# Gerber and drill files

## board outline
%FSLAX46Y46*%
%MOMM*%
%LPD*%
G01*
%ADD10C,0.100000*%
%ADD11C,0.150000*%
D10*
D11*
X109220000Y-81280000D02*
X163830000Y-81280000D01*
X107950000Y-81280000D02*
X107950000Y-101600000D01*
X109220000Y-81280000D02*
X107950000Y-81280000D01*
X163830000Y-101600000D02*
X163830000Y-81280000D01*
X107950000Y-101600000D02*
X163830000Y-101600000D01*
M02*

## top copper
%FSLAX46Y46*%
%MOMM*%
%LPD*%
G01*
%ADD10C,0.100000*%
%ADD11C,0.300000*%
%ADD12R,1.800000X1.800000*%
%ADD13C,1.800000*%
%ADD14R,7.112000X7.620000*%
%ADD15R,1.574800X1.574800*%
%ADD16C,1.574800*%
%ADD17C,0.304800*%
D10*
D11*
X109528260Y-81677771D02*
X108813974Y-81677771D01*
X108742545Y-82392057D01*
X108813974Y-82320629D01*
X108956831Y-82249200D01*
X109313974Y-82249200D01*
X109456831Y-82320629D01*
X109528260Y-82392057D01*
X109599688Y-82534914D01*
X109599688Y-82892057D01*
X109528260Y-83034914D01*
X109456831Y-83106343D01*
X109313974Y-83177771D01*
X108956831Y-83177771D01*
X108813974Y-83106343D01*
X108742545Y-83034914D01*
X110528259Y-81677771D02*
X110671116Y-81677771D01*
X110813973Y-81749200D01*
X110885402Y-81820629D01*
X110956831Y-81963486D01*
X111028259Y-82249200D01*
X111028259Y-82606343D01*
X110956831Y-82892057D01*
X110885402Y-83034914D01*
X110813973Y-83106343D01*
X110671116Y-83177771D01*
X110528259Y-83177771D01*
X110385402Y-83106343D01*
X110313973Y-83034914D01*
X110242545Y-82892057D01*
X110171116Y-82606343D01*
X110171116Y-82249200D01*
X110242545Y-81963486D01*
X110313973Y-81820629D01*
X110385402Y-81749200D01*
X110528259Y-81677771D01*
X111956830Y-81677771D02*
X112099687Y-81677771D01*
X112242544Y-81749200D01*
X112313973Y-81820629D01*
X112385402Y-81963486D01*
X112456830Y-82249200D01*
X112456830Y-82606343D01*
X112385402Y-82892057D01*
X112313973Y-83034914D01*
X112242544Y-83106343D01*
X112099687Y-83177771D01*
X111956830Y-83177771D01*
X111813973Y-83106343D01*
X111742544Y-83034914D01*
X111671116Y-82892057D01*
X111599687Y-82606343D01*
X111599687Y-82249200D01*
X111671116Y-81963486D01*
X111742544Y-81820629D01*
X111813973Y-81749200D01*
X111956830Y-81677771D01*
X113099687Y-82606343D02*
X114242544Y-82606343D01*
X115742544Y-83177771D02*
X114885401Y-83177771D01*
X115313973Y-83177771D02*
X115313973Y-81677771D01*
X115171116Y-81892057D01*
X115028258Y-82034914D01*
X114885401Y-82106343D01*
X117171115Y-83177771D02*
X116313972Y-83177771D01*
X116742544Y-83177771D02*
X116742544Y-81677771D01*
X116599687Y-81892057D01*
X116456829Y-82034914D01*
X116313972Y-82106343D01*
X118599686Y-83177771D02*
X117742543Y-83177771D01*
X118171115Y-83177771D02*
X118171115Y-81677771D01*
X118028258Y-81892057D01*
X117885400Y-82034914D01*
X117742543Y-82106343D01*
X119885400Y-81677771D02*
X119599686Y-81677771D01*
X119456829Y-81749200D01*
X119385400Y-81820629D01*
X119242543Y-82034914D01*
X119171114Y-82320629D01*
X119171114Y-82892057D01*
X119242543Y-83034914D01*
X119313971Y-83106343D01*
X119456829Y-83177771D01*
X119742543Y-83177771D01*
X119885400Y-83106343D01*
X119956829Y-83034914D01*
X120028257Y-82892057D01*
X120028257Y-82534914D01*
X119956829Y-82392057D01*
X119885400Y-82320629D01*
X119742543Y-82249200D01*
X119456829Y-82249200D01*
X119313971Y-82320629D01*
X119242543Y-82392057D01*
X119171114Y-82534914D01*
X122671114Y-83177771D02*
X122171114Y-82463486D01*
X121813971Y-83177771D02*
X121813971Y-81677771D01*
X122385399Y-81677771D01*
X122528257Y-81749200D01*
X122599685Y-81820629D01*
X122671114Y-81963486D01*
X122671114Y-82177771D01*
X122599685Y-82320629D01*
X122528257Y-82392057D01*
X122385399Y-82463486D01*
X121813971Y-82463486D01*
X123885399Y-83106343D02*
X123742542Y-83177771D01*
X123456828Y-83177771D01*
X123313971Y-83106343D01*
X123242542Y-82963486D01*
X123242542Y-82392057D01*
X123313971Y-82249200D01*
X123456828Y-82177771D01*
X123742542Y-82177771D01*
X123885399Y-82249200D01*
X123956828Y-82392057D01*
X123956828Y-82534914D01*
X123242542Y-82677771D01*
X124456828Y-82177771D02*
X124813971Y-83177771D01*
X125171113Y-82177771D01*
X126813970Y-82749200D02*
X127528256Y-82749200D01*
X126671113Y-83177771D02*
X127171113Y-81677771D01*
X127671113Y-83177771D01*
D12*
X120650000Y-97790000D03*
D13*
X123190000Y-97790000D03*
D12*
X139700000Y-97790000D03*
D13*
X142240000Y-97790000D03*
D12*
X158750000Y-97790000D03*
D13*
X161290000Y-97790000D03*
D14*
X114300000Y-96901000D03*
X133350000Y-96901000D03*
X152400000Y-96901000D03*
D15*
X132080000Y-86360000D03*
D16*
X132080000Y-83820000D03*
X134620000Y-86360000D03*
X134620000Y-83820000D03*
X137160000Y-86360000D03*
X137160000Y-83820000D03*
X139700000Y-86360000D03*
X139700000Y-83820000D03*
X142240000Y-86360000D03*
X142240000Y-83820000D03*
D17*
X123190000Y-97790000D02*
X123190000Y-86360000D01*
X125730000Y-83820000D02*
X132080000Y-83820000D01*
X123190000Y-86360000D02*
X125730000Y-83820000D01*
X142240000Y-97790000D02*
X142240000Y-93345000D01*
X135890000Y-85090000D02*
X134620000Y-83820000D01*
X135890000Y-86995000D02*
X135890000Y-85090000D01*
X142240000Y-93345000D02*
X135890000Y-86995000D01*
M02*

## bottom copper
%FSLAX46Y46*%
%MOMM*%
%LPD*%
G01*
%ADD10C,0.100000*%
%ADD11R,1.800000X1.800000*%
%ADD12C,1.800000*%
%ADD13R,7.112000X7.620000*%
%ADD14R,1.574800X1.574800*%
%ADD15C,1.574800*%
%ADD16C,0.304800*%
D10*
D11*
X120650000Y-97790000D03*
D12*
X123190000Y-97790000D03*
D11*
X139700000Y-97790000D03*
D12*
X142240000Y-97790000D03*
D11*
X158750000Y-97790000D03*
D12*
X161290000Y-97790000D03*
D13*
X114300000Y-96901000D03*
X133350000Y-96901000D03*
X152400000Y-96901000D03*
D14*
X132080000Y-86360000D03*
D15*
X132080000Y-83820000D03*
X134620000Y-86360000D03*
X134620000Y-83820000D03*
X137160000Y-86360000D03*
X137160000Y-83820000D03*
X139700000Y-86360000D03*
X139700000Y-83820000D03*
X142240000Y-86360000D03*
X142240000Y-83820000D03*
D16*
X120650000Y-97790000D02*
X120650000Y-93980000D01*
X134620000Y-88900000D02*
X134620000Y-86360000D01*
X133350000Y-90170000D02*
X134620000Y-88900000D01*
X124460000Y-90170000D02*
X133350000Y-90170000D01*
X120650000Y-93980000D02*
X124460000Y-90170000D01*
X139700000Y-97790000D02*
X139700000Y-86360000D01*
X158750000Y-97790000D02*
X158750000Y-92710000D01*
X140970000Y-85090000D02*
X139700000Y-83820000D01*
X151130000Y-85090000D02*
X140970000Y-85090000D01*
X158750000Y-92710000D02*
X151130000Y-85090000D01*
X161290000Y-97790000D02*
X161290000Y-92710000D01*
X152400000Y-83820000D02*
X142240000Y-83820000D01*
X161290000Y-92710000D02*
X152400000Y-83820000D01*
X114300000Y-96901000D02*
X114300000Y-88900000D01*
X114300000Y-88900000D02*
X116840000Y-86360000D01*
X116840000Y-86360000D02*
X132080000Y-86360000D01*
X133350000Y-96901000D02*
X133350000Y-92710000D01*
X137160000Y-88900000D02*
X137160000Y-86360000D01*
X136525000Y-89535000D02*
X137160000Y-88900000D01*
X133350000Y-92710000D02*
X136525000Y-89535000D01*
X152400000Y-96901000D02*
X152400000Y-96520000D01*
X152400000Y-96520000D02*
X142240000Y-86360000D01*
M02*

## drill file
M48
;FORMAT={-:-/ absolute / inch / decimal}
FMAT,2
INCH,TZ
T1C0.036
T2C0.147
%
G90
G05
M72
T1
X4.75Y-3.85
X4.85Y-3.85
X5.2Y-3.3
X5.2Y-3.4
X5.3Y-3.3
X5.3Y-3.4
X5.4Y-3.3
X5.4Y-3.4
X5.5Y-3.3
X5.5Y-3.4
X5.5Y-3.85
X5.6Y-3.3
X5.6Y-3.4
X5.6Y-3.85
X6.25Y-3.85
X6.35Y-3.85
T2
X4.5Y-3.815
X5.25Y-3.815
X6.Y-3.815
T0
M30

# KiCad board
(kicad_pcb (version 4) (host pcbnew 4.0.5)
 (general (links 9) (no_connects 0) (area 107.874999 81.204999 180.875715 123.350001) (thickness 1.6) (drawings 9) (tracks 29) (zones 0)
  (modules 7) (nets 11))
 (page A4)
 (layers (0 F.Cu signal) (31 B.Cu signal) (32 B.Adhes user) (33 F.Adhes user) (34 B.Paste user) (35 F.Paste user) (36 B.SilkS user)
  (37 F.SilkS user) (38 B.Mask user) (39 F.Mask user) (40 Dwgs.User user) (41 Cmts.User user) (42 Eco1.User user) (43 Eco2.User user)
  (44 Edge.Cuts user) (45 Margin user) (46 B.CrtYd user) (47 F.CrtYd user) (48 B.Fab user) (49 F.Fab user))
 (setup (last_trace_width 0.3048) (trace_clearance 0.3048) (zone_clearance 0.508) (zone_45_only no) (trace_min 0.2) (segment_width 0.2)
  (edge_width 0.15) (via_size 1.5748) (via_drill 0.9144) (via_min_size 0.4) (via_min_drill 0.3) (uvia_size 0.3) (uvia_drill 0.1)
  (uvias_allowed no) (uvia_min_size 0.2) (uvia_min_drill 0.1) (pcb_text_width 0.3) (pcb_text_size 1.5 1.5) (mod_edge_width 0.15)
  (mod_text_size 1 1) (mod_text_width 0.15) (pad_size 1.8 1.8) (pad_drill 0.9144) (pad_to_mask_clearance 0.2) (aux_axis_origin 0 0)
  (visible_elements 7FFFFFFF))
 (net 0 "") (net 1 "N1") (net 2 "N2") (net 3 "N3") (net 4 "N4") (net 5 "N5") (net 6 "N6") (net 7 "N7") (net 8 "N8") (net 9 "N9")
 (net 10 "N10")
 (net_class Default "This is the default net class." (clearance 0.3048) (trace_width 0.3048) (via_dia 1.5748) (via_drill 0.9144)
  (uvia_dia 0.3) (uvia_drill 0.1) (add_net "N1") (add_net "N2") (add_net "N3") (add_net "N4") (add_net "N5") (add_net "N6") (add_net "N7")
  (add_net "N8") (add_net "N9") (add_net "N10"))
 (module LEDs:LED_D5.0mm (layer F.Cu) (at 120.65 97.79)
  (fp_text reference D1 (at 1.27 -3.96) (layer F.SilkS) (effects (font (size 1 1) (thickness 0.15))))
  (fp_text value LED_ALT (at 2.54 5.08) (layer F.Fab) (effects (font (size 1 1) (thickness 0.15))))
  (pad 1 thru_hole rect (at 0 0) (size 1.8 1.8) (drill 0.9144) (layers *.Cu *.Mask) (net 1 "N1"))
  (pad 2 thru_hole circle (at 2.54 0) (size 1.8 1.8) (drill 0.9144) (layers *.Cu *.Mask) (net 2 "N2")))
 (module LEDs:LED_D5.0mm (layer F.Cu) (at 139.7 97.79)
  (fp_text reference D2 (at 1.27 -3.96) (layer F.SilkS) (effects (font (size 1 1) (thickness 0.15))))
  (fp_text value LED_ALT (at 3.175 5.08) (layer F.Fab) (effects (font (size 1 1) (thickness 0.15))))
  (pad 1 thru_hole rect (at 0 0) (size 1.8 1.8) (drill 0.9144) (layers *.Cu *.Mask) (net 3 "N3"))
  (pad 2 thru_hole circle (at 2.54 0) (size 1.8 1.8) (drill 0.9144) (layers *.Cu *.Mask) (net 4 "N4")))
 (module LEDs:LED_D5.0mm (layer F.Cu) (at 158.75 97.79)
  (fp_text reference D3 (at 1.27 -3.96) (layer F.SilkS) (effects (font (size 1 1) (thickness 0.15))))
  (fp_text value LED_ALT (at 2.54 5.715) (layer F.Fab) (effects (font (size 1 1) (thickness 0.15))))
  (pad 1 thru_hole rect (at 0 0) (size 1.8 1.8) (drill 0.9144) (layers *.Cu *.Mask) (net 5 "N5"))
  (pad 2 thru_hole circle (at 2.54 0) (size 1.8 1.8) (drill 0.9144) (layers *.Cu *.Mask) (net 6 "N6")))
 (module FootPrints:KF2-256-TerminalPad (layer F.Cu) (at 114.3 101.6)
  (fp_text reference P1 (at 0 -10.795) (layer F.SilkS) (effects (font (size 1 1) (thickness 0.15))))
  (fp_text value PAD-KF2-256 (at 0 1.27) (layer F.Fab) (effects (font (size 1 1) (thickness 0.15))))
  (pad 1 thru_hole rect (at 0 -4.699) (size 7.112 7.62) (drill 3.7338) (layers *.Cu *.Mask F.SilkS) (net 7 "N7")))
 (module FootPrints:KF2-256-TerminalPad (layer F.Cu) (at 133.35 101.6)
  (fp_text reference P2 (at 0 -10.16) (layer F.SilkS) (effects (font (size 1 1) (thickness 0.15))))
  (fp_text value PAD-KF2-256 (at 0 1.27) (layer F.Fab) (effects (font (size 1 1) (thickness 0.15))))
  (pad 1 thru_hole rect (at 0 -4.699) (size 7.112 7.62) (drill 3.7338) (layers *.Cu *.Mask F.SilkS) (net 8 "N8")))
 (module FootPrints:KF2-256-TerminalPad (layer F.Cu) (at 152.4 101.6)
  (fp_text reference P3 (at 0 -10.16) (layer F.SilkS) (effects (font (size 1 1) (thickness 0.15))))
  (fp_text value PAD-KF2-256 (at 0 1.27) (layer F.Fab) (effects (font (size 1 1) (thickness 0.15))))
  (pad 1 thru_hole rect (at 0 -4.699) (size 7.112 7.62) (drill 3.7338) (layers *.Cu *.Mask F.SilkS) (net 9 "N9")))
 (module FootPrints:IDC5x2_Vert (layer F.Cu) (at 137.16 85.09 180)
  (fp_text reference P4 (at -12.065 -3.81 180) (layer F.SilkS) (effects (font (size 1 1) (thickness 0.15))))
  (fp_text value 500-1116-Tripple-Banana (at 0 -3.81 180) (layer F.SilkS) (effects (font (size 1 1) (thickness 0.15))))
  (pad 1 thru_hole rect (at 5.08 -1.27 180) (size 1.5748 1.5748) (drill 0.9144) (layers *.Cu *.Mask F.SilkS) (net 7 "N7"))
  (pad 2 thru_hole circle (at 5.08 1.27 180) (size 1.5748 1.5748) (drill 0.9144) (layers *.Cu *.Mask F.SilkS) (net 2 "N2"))
  (pad 3 thru_hole circle (at 2.54 -1.27 180) (size 1.5748 1.5748) (drill 0.9144) (layers *.Cu *.Mask F.SilkS) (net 1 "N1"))
  (pad 4 thru_hole circle (at 2.54 1.27 180) (size 1.5748 1.5748) (drill 0.9144) (layers *.Cu *.Mask F.SilkS) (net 4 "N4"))
  (pad 5 thru_hole circle (at 0 -1.27 180) (size 1.5748 1.5748) (drill 0.9144) (layers *.Cu *.Mask F.SilkS) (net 8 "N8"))
  (pad 6 thru_hole circle (at 0 1.27 180) (size 1.5748 1.5748) (drill 0.9144) (layers *.Cu *.Mask F.SilkS) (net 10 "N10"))
  (pad 7 thru_hole circle (at -2.54 -1.27 180) (size 1.5748 1.5748) (drill 0.9144) (layers *.Cu *.Mask F.SilkS) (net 3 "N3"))
  (pad 8 thru_hole circle (at -2.54 1.27 180) (size 1.5748 1.5748) (drill 0.9144) (layers *.Cu *.Mask F.SilkS) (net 5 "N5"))
  (pad 9 thru_hole circle (at -5.08 -1.27 180) (size 1.5748 1.5748) (drill 0.9144) (layers *.Cu *.Mask F.SilkS) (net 9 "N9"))
  (pad 10 thru_hole circle (at -5.08 1.27 180) (size 1.5748 1.5748) (drill 0.9144) (layers *.Cu *.Mask F.SilkS) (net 6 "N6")))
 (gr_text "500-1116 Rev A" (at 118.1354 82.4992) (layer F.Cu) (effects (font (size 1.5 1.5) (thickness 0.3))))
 (gr_line (start 109.22 81.28) (end 163.83 81.28) (angle 90) (layer Edge.Cuts) (width 0.15))
 (gr_line (start 107.95 81.28) (end 107.95 101.6) (angle 90) (layer Edge.Cuts) (width 0.15))
 (gr_line (start 109.22 81.28) (end 107.95 81.28) (angle 90) (layer Edge.Cuts) (width 0.15))
 (gr_line (start 163.83 101.6) (end 163.83 81.28) (angle 90) (layer Edge.Cuts) (width 0.15))
 (gr_line (start 107.95 101.6) (end 163.83 101.6) (angle 90) (layer Edge.Cuts) (width 0.15))
 (segment (start 120.65 97.79) (end 120.65 93.98) (width 0.3048) (layer B.Cu) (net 1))
 (segment (start 134.62 88.9) (end 134.62 86.36) (width 0.3048) (layer B.Cu) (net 1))
 (segment (start 133.35 90.17) (end 134.62 88.9) (width 0.3048) (layer B.Cu) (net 1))
 (segment (start 124.46 90.17) (end 133.35 90.17) (width 0.3048) (layer B.Cu) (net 1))
 (segment (start 120.65 93.98) (end 124.46 90.17) (width 0.3048) (layer B.Cu) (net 1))
 (segment (start 123.19 97.79) (end 123.19 86.36) (width 0.3048) (layer F.Cu) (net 2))
 (segment (start 125.73 83.82) (end 132.08 83.82) (width 0.3048) (layer F.Cu) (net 2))
 (segment (start 123.19 86.36) (end 125.73 83.82) (width 0.3048) (layer F.Cu) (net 2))
 (segment (start 139.7 97.79) (end 139.7 86.36) (width 0.3048) (layer B.Cu) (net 3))
 (segment (start 142.24 97.79) (end 142.24 93.345) (width 0.3048) (layer F.Cu) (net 4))
 (segment (start 135.89 85.09) (end 134.62 83.82) (width 0.3048) (layer F.Cu) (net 4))
 (segment (start 135.89 86.995) (end 135.89 85.09) (width 0.3048) (layer F.Cu) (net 4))
 (segment (start 142.24 93.345) (end 135.89 86.995) (width 0.3048) (layer F.Cu) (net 4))
 (segment (start 158.75 97.79) (end 158.75 92.71) (width 0.3048) (layer B.Cu) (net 5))
 (segment (start 140.97 85.09) (end 139.7 83.82) (width 0.3048) (layer B.Cu) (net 5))
 (segment (start 151.13 85.09) (end 140.97 85.09) (width 0.3048) (layer B.Cu) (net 5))
 (segment (start 158.75 92.71) (end 151.13 85.09) (width 0.3048) (layer B.Cu) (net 5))
 (segment (start 161.29 97.79) (end 161.29 92.71) (width 0.3048) (layer B.Cu) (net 6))
 (segment (start 152.4 83.82) (end 142.24 83.82) (width 0.3048) (layer B.Cu) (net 6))
 (segment (start 161.29 92.71) (end 152.4 83.82) (width 0.3048) (layer B.Cu) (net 6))
 (segment (start 114.3 96.901) (end 114.3 88.9) (width 0.3048) (layer B.Cu) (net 7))
 (segment (start 114.3 88.9) (end 116.84 86.36) (width 0.3048) (layer B.Cu) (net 7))
 (segment (start 116.84 86.36) (end 132.08 86.36) (width 0.3048) (layer B.Cu) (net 7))
 (segment (start 133.35 96.901) (end 133.35 92.71) (width 0.3048) (layer B.Cu) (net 8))
 (segment (start 137.16 88.9) (end 137.16 86.36) (width 0.3048) (layer B.Cu) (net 8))
 (segment (start 136.525 89.535) (end 137.16 88.9) (width 0.3048) (layer B.Cu) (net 8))
 (segment (start 133.35 92.71) (end 136.525 89.535) (width 0.3048) (layer B.Cu) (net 8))
 (segment (start 152.4 96.901) (end 152.4 96.52) (width 0.3048) (layer B.Cu) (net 9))
 (segment (start 152.4 96.52) (end 142.24 86.36) (width 0.3048) (layer B.Cu) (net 9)))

